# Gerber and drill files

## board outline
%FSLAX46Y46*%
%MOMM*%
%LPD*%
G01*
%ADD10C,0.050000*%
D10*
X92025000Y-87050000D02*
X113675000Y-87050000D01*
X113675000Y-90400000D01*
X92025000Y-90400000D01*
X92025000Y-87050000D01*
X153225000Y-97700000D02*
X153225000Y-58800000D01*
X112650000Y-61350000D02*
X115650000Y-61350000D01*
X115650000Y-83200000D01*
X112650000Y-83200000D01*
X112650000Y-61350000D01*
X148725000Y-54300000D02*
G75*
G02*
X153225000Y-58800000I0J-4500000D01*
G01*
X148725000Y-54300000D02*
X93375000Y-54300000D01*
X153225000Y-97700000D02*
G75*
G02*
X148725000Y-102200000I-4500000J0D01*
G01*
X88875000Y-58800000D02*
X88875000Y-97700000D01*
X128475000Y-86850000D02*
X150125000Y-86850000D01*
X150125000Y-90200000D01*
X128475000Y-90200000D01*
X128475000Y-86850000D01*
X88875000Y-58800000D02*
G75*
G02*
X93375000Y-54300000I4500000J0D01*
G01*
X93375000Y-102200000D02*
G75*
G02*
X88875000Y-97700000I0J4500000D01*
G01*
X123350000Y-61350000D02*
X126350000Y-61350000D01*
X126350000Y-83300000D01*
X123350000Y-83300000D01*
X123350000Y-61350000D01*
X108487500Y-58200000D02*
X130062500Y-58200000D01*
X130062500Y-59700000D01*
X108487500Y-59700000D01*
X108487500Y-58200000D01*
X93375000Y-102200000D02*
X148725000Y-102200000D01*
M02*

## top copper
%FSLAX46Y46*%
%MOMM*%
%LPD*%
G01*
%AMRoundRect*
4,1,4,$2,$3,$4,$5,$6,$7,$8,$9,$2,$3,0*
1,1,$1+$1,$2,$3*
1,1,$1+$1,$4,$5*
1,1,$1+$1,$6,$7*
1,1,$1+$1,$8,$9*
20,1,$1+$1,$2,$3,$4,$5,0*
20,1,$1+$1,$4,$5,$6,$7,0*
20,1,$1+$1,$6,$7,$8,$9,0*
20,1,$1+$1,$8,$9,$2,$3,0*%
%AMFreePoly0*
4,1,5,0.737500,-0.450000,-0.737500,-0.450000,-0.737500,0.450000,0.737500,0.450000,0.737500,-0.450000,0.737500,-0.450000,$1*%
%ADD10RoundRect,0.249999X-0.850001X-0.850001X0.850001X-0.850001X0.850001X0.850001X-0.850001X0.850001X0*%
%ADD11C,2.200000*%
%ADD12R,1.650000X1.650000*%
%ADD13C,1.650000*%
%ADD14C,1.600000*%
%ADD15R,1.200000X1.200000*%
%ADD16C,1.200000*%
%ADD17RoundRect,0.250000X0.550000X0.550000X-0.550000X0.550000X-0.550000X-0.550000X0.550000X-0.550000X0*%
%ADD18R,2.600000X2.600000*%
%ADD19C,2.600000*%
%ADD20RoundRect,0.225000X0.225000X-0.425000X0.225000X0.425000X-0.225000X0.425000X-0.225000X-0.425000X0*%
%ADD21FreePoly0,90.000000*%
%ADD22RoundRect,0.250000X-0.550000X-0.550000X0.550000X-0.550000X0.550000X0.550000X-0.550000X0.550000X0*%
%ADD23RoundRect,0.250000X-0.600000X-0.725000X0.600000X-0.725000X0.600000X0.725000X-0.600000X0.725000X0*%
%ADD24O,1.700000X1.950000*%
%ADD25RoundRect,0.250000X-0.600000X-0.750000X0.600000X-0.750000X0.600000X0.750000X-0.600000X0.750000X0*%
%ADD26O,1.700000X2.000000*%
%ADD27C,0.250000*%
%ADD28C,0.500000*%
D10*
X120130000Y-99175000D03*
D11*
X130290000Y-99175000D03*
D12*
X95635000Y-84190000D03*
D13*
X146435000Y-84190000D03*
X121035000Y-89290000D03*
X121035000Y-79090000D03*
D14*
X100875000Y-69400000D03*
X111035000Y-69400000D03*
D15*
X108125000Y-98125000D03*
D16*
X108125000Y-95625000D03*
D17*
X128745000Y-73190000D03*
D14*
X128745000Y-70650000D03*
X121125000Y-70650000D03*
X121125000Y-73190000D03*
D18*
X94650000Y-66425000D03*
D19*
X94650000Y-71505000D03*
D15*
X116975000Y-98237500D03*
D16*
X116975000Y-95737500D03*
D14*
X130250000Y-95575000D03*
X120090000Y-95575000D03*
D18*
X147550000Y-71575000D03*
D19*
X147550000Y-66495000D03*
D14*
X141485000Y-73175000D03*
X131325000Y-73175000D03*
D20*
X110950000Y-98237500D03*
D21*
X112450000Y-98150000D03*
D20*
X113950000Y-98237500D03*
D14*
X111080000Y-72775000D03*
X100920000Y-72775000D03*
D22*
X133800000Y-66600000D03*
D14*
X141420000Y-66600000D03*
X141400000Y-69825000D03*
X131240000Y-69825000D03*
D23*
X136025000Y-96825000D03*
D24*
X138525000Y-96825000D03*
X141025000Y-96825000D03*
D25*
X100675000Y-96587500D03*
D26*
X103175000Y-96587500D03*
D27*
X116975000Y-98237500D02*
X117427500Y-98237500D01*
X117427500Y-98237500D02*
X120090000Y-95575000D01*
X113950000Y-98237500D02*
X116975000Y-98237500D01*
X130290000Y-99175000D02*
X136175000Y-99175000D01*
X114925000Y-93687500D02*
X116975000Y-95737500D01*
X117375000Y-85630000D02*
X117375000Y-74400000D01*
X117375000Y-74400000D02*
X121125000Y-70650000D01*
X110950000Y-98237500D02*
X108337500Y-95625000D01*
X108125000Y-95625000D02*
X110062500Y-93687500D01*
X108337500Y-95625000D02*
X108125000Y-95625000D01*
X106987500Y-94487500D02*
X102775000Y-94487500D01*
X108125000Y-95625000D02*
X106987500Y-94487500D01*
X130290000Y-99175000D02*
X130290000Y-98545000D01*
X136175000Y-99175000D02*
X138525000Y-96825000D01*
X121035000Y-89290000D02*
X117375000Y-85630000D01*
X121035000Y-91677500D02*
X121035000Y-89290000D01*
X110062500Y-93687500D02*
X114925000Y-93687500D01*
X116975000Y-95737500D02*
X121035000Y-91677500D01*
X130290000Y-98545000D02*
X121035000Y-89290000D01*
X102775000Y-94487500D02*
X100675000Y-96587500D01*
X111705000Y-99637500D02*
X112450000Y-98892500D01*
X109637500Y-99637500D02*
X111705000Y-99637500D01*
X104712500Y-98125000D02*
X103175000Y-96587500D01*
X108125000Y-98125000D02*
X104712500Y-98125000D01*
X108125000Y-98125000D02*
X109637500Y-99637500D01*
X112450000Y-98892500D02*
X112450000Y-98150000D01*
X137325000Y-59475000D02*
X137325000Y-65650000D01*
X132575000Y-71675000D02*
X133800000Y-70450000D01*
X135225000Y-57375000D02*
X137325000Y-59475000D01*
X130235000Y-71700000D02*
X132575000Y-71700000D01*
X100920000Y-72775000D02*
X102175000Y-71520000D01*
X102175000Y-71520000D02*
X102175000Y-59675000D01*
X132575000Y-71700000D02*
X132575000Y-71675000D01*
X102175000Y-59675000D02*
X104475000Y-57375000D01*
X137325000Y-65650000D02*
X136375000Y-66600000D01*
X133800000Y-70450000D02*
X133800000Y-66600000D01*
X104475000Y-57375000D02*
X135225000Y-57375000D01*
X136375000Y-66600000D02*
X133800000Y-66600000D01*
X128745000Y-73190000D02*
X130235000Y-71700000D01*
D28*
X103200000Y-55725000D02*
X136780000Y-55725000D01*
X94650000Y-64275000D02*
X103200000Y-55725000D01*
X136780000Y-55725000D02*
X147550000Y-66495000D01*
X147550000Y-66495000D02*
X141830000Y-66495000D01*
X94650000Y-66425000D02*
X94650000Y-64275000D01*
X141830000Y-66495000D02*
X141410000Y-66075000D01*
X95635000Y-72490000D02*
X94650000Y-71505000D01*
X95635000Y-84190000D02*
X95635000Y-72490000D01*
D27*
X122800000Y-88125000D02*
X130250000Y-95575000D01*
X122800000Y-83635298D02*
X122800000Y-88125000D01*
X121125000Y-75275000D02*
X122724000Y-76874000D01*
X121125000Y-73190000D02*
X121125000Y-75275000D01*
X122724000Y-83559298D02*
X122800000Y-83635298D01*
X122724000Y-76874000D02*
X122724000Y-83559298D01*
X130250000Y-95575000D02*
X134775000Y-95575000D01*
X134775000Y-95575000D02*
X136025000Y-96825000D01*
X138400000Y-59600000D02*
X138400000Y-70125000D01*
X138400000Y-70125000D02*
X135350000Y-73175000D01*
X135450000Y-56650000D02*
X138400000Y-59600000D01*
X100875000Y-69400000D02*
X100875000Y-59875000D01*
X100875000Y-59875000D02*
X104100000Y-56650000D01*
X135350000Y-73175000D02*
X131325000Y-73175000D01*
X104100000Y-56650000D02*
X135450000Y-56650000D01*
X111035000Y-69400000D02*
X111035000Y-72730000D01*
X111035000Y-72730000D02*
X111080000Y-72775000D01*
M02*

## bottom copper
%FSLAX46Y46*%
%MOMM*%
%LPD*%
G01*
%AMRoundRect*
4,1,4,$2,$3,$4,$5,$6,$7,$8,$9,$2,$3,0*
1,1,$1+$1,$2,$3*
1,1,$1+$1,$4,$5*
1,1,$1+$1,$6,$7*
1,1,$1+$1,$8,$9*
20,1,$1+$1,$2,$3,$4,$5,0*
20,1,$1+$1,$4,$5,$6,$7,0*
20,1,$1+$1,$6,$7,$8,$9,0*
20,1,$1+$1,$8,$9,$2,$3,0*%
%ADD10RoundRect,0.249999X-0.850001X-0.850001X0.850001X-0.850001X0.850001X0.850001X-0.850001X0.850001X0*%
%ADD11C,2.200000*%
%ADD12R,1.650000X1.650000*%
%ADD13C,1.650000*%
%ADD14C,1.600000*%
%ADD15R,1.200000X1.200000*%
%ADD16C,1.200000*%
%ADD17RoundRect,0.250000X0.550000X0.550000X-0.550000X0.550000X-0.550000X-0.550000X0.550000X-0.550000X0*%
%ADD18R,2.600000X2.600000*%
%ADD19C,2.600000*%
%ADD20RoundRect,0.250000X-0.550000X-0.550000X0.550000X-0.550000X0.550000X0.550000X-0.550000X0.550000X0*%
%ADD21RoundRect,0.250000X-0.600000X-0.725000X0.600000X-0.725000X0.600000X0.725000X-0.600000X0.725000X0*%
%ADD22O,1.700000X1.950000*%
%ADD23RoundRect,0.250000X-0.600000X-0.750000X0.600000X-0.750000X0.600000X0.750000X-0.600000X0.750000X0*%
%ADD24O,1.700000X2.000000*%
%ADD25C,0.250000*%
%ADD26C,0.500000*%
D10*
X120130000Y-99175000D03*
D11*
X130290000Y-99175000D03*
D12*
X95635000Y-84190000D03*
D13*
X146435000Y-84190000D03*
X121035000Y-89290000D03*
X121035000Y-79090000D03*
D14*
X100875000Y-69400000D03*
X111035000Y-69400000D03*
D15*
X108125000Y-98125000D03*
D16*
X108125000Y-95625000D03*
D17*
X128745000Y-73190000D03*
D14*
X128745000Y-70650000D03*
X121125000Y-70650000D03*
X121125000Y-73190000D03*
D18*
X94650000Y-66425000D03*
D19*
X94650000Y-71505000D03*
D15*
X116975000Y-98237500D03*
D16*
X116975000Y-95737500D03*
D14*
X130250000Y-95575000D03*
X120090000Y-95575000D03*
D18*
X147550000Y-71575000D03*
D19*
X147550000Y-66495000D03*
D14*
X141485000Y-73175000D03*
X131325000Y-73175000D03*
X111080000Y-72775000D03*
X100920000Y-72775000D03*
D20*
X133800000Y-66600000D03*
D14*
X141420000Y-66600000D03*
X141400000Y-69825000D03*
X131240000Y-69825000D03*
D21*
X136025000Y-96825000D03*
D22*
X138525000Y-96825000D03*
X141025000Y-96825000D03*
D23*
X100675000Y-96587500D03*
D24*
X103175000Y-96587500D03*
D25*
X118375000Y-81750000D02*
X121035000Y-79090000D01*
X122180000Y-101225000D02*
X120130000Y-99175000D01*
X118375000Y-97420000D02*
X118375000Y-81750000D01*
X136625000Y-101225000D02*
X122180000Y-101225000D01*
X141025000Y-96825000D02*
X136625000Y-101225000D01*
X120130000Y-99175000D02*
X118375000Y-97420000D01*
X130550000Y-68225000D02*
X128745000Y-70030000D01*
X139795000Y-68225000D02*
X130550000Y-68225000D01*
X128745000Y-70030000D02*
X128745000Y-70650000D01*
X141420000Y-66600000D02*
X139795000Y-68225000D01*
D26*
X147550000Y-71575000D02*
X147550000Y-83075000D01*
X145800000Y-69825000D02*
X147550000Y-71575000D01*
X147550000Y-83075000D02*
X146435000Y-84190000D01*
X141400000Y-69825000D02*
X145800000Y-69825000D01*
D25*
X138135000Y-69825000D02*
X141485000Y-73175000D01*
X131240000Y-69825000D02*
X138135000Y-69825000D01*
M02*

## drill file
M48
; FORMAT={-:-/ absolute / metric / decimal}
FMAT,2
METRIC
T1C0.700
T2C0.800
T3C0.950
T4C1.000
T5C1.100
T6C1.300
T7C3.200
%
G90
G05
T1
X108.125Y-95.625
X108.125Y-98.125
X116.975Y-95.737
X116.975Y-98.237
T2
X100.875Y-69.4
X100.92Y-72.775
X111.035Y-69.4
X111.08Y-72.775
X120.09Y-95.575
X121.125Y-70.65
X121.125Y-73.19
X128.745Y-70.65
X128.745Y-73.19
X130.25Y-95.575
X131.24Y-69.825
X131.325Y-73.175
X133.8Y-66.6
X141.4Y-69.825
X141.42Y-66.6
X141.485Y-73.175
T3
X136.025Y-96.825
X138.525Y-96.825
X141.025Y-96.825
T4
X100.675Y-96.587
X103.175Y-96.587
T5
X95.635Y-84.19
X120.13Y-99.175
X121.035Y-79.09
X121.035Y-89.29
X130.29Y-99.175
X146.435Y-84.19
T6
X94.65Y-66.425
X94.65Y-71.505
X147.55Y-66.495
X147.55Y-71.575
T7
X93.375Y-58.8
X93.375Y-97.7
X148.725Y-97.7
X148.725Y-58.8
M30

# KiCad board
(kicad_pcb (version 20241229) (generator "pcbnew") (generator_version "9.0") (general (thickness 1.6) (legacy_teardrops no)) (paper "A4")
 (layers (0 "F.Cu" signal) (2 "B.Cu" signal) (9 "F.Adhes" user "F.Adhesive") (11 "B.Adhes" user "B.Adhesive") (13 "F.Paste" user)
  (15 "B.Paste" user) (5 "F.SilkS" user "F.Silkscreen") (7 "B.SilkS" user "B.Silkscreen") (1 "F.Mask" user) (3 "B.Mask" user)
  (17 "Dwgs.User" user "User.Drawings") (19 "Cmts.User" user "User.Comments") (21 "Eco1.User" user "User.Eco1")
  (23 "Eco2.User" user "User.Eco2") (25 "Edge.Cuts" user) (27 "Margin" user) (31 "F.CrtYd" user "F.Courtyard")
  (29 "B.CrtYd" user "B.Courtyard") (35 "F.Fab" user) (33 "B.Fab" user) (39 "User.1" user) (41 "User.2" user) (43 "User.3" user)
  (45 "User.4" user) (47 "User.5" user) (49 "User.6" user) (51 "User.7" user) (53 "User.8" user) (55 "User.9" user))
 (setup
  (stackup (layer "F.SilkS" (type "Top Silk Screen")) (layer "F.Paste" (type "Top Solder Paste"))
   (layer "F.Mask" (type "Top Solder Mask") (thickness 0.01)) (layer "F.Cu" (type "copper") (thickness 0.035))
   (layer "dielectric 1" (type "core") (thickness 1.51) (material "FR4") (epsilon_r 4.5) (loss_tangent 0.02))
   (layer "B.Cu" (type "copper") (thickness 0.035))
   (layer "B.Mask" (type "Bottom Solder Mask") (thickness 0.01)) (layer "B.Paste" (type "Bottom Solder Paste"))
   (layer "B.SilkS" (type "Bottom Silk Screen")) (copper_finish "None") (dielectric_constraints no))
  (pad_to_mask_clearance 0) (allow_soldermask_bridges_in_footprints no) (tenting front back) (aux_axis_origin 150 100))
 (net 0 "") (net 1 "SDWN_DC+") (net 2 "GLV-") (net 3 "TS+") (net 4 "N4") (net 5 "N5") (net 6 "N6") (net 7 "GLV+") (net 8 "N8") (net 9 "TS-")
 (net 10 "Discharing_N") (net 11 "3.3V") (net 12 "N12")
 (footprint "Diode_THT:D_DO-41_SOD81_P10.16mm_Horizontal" (layer "F.Cu") (at 120.13 99.175)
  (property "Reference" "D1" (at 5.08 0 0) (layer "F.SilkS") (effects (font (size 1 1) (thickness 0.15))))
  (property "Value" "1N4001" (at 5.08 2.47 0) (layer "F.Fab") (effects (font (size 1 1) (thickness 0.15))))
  (pad "1" thru_hole roundrect (at 0 0) (size 2.2 2.2) (drill 1.1) (layers "*.Cu" "*.Mask") (remove_unused_layers no)
   (roundrect_rratio 0.113636) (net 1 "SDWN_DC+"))
  (pad "2" thru_hole circle (at 10.16 0) (size 2.2 2.2) (drill 1.1) (layers "*.Cu" "*.Mask") (remove_unused_layers no) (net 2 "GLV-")))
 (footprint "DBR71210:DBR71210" (layer "F.Cu") (at 95.635 84.19)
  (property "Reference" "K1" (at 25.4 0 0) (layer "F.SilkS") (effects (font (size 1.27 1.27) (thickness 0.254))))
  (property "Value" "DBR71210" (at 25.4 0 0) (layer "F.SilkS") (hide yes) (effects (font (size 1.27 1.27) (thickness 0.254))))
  (pad "1" thru_hole rect (at 0 0) (size 1.65 1.65) (drill 1.1) (layers "*.Cu" "*.Mask") (remove_unused_layers no) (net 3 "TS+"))
  (pad "2" thru_hole circle (at 50.8 0) (size 1.65 1.65) (drill 1.1) (layers "*.Cu" "*.Mask") (remove_unused_layers no) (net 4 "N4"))
  (pad "3" thru_hole circle (at 25.4 5.1) (size 1.65 1.65) (drill 1.1) (layers "*.Cu" "*.Mask") (remove_unused_layers no) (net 2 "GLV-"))
  (pad "4" thru_hole circle (at 25.4 -5.1) (size 1.65 1.65) (drill 1.1) (layers "*.Cu" "*.Mask") (remove_unused_layers no)
   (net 1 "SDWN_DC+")))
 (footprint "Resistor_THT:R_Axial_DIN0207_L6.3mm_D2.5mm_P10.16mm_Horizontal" (layer "F.Cu") (at 100.875 69.4)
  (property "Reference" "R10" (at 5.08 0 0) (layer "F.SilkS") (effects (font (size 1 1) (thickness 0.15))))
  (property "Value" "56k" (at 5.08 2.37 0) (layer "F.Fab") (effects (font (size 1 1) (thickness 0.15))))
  (pad "1" thru_hole circle (at 0 0) (size 1.6 1.6) (drill 0.8) (layers "*.Cu" "*.Mask") (remove_unused_layers no) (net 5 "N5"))
  (pad "2" thru_hole circle (at 10.16 0) (size 1.6 1.6) (drill 0.8) (layers "*.Cu" "*.Mask") (remove_unused_layers no) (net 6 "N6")))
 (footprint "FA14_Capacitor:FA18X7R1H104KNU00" (layer "F.Cu") (at 108.125 98.125 90)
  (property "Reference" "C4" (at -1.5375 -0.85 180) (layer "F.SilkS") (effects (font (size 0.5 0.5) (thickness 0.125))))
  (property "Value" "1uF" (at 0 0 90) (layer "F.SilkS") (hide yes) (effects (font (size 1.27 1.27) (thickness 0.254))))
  (pad "1" thru_hole rect (at 0 0 90) (size 1.2 1.2) (drill 0.7) (layers "*.Cu" "*.Mask") (remove_unused_layers no) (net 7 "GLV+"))
  (pad "2" thru_hole circle (at 2.5 0 90) (size 1.2 1.2) (drill 0.7) (layers "*.Cu" "*.Mask") (remove_unused_layers no) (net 2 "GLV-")))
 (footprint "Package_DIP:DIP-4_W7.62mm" (layer "F.Cu") (at 128.745 73.19 180)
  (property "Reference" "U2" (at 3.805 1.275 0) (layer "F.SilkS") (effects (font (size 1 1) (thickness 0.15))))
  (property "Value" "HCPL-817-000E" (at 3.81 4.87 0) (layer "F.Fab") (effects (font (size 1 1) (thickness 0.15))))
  (pad "1" thru_hole roundrect (at 0 0 180) (size 1.6 1.6) (drill 0.8) (layers "*.Cu" "*.Mask") (remove_unused_layers no)
   (roundrect_rratio 0.15625) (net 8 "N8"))
  (pad "2" thru_hole circle (at 0 2.54 180) (size 1.6 1.6) (drill 0.8) (layers "*.Cu" "*.Mask") (remove_unused_layers no) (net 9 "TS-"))
  (pad "3" thru_hole circle (at 7.62 2.54 180) (size 1.6 1.6) (drill 0.8) (layers "*.Cu" "*.Mask") (remove_unused_layers no) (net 2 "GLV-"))
  (pad "4" thru_hole circle (at 7.62 0 180) (size 1.6 1.6) (drill 0.8) (layers "*.Cu" "*.Mask") (remove_unused_layers no)
   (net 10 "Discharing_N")))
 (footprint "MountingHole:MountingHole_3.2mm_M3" (layer "F.Cu") (at 93.374998 58.799998)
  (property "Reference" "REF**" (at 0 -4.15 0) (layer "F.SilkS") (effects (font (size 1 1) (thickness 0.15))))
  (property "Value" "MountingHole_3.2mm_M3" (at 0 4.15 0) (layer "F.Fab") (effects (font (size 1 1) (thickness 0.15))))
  (pad "" np_thru_hole circle (at 0 0) (size 3.2 3.2) (drill 3.2) (layers "*.Cu" "*.Mask")))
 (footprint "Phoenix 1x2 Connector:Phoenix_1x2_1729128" (layer "F.Cu") (at 94.65 66.425 -90)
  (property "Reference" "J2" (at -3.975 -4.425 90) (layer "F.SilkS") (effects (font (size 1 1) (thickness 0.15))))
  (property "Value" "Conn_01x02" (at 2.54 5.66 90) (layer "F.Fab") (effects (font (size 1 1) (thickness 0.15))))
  (pad "1" thru_hole rect (at 0 0 270) (size 2.6 2.6) (drill 1.3) (layers "*.Cu" "*.Mask") (remove_unused_layers no) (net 9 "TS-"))
  (pad "2" thru_hole circle (at 5.08 0 270) (size 2.6 2.6) (drill 1.3) (layers "*.Cu" "*.Mask") (remove_unused_layers no) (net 3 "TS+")))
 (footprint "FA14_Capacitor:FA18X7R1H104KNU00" (layer "F.Cu") (at 116.975 98.2375 90)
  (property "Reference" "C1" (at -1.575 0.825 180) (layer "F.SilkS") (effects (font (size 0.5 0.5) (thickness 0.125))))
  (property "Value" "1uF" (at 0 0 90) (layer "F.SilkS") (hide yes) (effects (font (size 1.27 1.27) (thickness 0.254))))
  (pad "1" thru_hole rect (at 0 0 90) (size 1.2 1.2) (drill 0.7) (layers "*.Cu" "*.Mask") (remove_unused_layers no) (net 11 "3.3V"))
  (pad "2" thru_hole circle (at 2.5 0 90) (size 1.2 1.2) (drill 0.7) (layers "*.Cu" "*.Mask") (remove_unused_layers no) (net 2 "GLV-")))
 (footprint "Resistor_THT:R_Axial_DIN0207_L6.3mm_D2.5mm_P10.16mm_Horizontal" (layer "F.Cu") (at 130.25 95.575 180)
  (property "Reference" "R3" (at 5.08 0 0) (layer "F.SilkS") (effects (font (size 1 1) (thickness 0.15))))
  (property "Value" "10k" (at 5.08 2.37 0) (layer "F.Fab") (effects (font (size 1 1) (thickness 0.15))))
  (pad "1" thru_hole circle (at 0 0 180) (size 1.6 1.6) (drill 0.8) (layers "*.Cu" "*.Mask") (remove_unused_layers no)
   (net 10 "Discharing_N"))
  (pad "2" thru_hole circle (at 10.16 0 180) (size 1.6 1.6) (drill 0.8) (layers "*.Cu" "*.Mask") (remove_unused_layers no) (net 11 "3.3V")))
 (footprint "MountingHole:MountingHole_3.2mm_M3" (layer "F.Cu") (at 148.725002 58.799998)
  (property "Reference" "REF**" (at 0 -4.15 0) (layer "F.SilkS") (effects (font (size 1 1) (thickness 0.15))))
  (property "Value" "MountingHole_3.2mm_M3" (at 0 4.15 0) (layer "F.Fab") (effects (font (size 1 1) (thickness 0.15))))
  (pad "" np_thru_hole circle (at 0 0) (size 3.2 3.2) (drill 3.2) (layers "*.Cu" "*.Mask")))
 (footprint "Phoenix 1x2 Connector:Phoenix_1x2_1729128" (layer "F.Cu") (at 147.55 71.575 90)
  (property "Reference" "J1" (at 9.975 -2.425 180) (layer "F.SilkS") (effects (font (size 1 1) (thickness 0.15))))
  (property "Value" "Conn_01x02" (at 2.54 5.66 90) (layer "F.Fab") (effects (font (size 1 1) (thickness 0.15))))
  (pad "1" thru_hole rect (at 0 0 90) (size 2.6 2.6) (drill 1.3) (layers "*.Cu" "*.Mask") (remove_unused_layers no) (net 4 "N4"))
  (pad "2" thru_hole circle (at 5.08 0 90) (size 2.6 2.6) (drill 1.3) (layers "*.Cu" "*.Mask") (remove_unused_layers no) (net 9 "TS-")))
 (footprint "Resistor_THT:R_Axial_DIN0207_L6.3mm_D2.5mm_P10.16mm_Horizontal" (layer "F.Cu") (at 141.485 73.175 180)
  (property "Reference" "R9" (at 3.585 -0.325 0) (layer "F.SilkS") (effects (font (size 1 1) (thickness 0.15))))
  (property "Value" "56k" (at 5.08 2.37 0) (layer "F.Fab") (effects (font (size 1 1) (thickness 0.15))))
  (pad "1" thru_hole circle (at 0 0 180) (size 1.6 1.6) (drill 0.8) (layers "*.Cu" "*.Mask") (remove_unused_layers no) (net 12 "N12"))
  (pad "2" thru_hole circle (at 10.16 0 180) (size 1.6 1.6) (drill 0.8) (layers "*.Cu" "*.Mask") (remove_unused_layers no) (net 5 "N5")))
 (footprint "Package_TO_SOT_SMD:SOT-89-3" (layer "F.Cu") (at 112.45 96.2875 90)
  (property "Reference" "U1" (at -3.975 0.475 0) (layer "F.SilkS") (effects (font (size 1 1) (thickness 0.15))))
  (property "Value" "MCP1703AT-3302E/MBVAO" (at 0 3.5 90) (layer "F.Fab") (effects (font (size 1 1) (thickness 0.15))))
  (pad "1" smd roundrect (at -1.95 -1.5 90) (size 1.3 0.9) (layers "F.Cu" "F.Mask" "F.Paste") (roundrect_rratio 0.25) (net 2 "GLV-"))
  (pad "2" smd custom (at -1.8625 0 90) (size 1.475 0.9) (layers "F.Cu" "F.Mask" "F.Paste") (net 7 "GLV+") (zone_connect 2)
   (thermal_bridge_angle 45) (options (clearance outline) (anchor rect)) (primitives))
  (pad "3" smd roundrect (at -1.95 1.5 90) (size 1.3 0.9) (layers "F.Cu" "F.Mask" "F.Paste") (roundrect_rratio 0.25) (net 11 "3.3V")))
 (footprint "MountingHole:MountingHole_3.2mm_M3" (layer "F.Cu") (at 93.375 97.7)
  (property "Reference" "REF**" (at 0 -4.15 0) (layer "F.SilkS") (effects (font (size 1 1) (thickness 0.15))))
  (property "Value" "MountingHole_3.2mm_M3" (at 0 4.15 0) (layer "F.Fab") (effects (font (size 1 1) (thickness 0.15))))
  (pad "" np_thru_hole circle (at 0 0) (size 3.2 3.2) (drill 3.2) (layers "*.Cu" "*.Mask")))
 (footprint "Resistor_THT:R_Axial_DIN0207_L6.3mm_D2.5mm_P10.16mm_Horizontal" (layer "F.Cu") (at 111.08 72.775 180)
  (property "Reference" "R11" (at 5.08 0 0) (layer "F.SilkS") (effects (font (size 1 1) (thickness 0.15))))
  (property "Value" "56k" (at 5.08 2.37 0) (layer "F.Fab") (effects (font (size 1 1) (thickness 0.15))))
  (pad "1" thru_hole circle (at 0 0 180) (size 1.6 1.6) (drill 0.8) (layers "*.Cu" "*.Mask") (remove_unused_layers no) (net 6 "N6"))
  (pad "2" thru_hole circle (at 10.16 0 180) (size 1.6 1.6) (drill 0.8) (layers "*.Cu" "*.Mask") (remove_unused_layers no) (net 8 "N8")))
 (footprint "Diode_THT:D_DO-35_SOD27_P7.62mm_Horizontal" (layer "F.Cu") (at 133.8 66.6)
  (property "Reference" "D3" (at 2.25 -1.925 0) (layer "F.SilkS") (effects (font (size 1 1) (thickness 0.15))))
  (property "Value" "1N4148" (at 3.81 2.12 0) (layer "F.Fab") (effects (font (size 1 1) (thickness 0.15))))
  (pad "1" thru_hole roundrect (at 0 0) (size 1.6 1.6) (drill 0.8) (layers "*.Cu" "*.Mask") (remove_unused_layers no)
   (roundrect_rratio 0.15625) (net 8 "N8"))
  (pad "2" thru_hole circle (at 7.62 0) (size 1.6 1.6) (drill 0.8) (layers "*.Cu" "*.Mask") (remove_unused_layers no) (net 9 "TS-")))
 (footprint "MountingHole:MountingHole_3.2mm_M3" (layer "F.Cu") (at 148.725 97.700002)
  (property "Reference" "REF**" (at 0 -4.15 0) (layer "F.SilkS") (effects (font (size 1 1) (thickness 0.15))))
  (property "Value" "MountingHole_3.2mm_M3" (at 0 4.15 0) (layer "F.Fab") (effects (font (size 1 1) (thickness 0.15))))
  (pad "" np_thru_hole circle (at 0 0) (size 3.2 3.2) (drill 3.2) (layers "*.Cu" "*.Mask")))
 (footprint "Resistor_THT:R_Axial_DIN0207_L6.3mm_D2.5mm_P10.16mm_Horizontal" (layer "F.Cu") (at 141.4 69.825 180)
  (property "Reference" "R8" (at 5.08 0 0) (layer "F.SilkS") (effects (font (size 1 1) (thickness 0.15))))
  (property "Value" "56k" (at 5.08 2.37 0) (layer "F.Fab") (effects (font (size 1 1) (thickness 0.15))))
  (pad "1" thru_hole circle (at 0 0 180) (size 1.6 1.6) (drill 0.8) (layers "*.Cu" "*.Mask") (remove_unused_layers no) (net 4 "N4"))
  (pad "2" thru_hole circle (at 10.16 0 180) (size 1.6 1.6) (drill 0.8) (layers "*.Cu" "*.Mask") (remove_unused_layers no) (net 12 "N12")))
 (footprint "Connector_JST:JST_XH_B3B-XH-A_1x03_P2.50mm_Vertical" (layer "F.Cu") (at 136.025 96.825)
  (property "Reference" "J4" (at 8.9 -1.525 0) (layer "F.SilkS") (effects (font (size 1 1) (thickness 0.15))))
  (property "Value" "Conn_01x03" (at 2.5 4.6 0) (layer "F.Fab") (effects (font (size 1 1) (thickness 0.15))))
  (pad "1" thru_hole roundrect (at 0 0) (size 1.7 1.95) (drill 0.95) (layers "*.Cu" "*.Mask") (remove_unused_layers no)
   (roundrect_rratio 0.147059) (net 10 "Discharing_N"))
  (pad "2" thru_hole oval (at 2.5 0) (size 1.7 1.95) (drill 0.95) (layers "*.Cu" "*.Mask") (remove_unused_layers no) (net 2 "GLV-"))
  (pad "3" thru_hole oval (at 5 0) (size 1.7 1.95) (drill 0.95) (layers "*.Cu" "*.Mask") (remove_unused_layers no) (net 1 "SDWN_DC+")))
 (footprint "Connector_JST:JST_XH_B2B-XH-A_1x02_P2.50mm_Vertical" (layer "F.Cu") (at 100.675 96.5875)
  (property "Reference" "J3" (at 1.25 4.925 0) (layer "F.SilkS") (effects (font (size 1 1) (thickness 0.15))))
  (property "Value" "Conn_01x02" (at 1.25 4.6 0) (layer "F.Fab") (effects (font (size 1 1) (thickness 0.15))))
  (pad "1" thru_hole roundrect (at 0 0) (size 1.7 2) (drill 1) (layers "*.Cu" "*.Mask") (remove_unused_layers no)
   (roundrect_rratio 0.147059) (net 2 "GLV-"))
  (pad "2" thru_hole oval (at 2.5 0) (size 1.7 2) (drill 1) (layers "*.Cu" "*.Mask") (remove_unused_layers no) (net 7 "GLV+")))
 (gr_rect (start 92.025 87.05) (end 113.675 90.4) (stroke (width 0.05) (type default)) (fill no) (layer "Edge.Cuts"))
 (gr_line (start 153.225 97.7) (end 153.225 58.8) (stroke (width 0.05) (type default)) (layer "Edge.Cuts"))
 (gr_rect (start 112.65 61.35) (end 115.65 83.2) (stroke (width 0.05) (type default)) (fill no) (layer "Edge.Cuts"))
 (gr_arc (start 148.725 54.3) (mid 151.906981 55.618019) (end 153.225 58.8) (stroke (width 0.05) (type default)) (layer "Edge.Cuts"))
 (gr_line (start 148.725 54.3) (end 93.375 54.3) (stroke (width 0.05) (type default)) (layer "Edge.Cuts"))
 (gr_arc (start 153.225 97.7) (mid 151.906981 100.881981) (end 148.725 102.2) (stroke (width 0.05) (type default)) (layer "Edge.Cuts"))
 (gr_line (start 88.875 58.8) (end 88.875 97.7) (stroke (width 0.05) (type default)) (layer "Edge.Cuts"))
 (gr_rect (start 128.475 86.85) (end 150.125 90.2) (stroke (width 0.05) (type default)) (fill no) (layer "Edge.Cuts"))
 (gr_arc (start 88.875 58.8) (mid 90.193019 55.618019) (end 93.375 54.3) (stroke (width 0.05) (type default)) (layer "Edge.Cuts"))
 (gr_arc (start 93.375 102.2) (mid 90.193019 100.881981) (end 88.875 97.7) (stroke (width 0.05) (type default)) (layer "Edge.Cuts"))
 (gr_rect (start 123.35 61.35) (end 126.35 83.3) (stroke (width 0.05) (type default)) (fill no) (layer "Edge.Cuts"))
 (gr_rect (start 108.4875 58.2) (end 130.0625 59.7) (stroke (width 0.05) (type default)) (fill no) (layer "Edge.Cuts"))
 (gr_line (start 93.375 102.2) (end 148.725 102.2) (stroke (width 0.05) (type default)) (layer "Edge.Cuts"))
 (segment (start 116.975 98.2375) (end 117.4275 98.2375) (width 0.25) (layer "F.Cu") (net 11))
 (segment (start 117.4275 98.2375) (end 120.09 95.575) (width 0.25) (layer "F.Cu") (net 11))
 (segment (start 113.95 98.2375) (end 116.975 98.2375) (width 0.25) (layer "F.Cu") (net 11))
 (segment (start 130.29 99.175) (end 136.175 99.175) (width 0.25) (layer "F.Cu") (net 2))
 (segment (start 114.925 93.6875) (end 116.975 95.7375) (width 0.25) (layer "F.Cu") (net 2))
 (segment (start 117.375 85.63) (end 117.375 74.4) (width 0.25) (layer "F.Cu") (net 2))
 (segment (start 117.375 74.4) (end 121.125 70.65) (width 0.25) (layer "F.Cu") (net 2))
 (segment (start 110.95 98.2375) (end 108.3375 95.625) (width 0.25) (layer "F.Cu") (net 2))
 (segment (start 108.125 95.625) (end 110.0625 93.6875) (width 0.25) (layer "F.Cu") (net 2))
 (segment (start 108.3375 95.625) (end 108.125 95.625) (width 0.25) (layer "F.Cu") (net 2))
 (segment (start 106.9875 94.4875) (end 102.775 94.4875) (width 0.25) (layer "F.Cu") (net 2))
 (segment (start 108.125 95.625) (end 106.9875 94.4875) (width 0.25) (layer "F.Cu") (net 2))
 (segment (start 130.29 99.175) (end 130.29 98.545) (width 0.25) (layer "F.Cu") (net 2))
 (segment (start 136.175 99.175) (end 138.525 96.825) (width 0.25) (layer "F.Cu") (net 2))
 (segment (start 121.035 89.29) (end 117.375 85.63) (width 0.25) (layer "F.Cu") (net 2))
 (segment (start 121.035 91.6775) (end 121.035 89.29) (width 0.25) (layer "F.Cu") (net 2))
 (segment (start 110.0625 93.6875) (end 114.925 93.6875) (width 0.25) (layer "F.Cu") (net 2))
 (segment (start 116.975 95.7375) (end 121.035 91.6775) (width 0.25) (layer "F.Cu") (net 2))
 (segment (start 130.29 98.545) (end 121.035 89.29) (width 0.25) (layer "F.Cu") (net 2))
 (segment (start 102.775 94.4875) (end 100.675 96.5875) (width 0.25) (layer "F.Cu") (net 2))
 (segment (start 111.705 99.6375) (end 112.45 98.8925) (width 0.25) (layer "F.Cu") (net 7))
 (segment (start 109.6375 99.6375) (end 111.705 99.6375) (width 0.25) (layer "F.Cu") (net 7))
 (segment (start 104.7125 98.125) (end 103.175 96.5875) (width 0.25) (layer "F.Cu") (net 7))
 (segment (start 108.125 98.125) (end 104.7125 98.125) (width 0.25) (layer "F.Cu") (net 7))
 (segment (start 108.125 98.125) (end 109.6375 99.6375) (width 0.25) (layer "F.Cu") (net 7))
 (segment (start 112.45 98.8925) (end 112.45 98.15) (width 0.25) (layer "F.Cu") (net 7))
 (segment (start 118.375 81.75) (end 121.035 79.09) (width 0.25) (layer "B.Cu") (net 1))
 (segment (start 122.18 101.225) (end 120.13 99.175) (width 0.25) (layer "B.Cu") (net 1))
 (segment (start 118.375 97.42) (end 118.375 81.75) (width 0.25) (layer "B.Cu") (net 1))
 (segment (start 136.625 101.225) (end 122.18 101.225) (width 0.25) (layer "B.Cu") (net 1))
 (segment (start 141.025 96.825) (end 136.625 101.225) (width 0.25) (layer "B.Cu") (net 1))
 (segment (start 120.13 99.175) (end 118.375 97.42) (width 0.25) (layer "B.Cu") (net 1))
 (segment (start 137.325 59.475) (end 137.325 65.65) (width 0.25) (layer "F.Cu") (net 8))
 (segment (start 132.575 71.675) (end 133.8 70.45) (width 0.25) (layer "F.Cu") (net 8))
 (segment (start 135.225 57.375) (end 137.325 59.475) (width 0.25) (layer "F.Cu") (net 8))
 (segment (start 130.235 71.7) (end 132.575 71.7) (width 0.25) (layer "F.Cu") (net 8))
 (segment (start 100.92 72.775) (end 102.175 71.52) (width 0.25) (layer "F.Cu") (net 8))
 (segment (start 102.175 71.52) (end 102.175 59.675) (width 0.25) (layer "F.Cu") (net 8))
 (segment (start 132.575 71.7) (end 132.575 71.675) (width 0.25) (layer "F.Cu") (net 8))
 (segment (start 102.175 59.675) (end 104.475 57.375) (width 0.25) (layer "F.Cu") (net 8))
 (segment (start 137.325 65.65) (end 136.375 66.6) (width 0.25) (layer "F.Cu") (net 8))
 (segment (start 133.8 70.45) (end 133.8 66.6) (width 0.25) (layer "F.Cu") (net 8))
 (segment (start 104.475 57.375) (end 135.225 57.375) (width 0.25) (layer "F.Cu") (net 8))
 (segment (start 136.375 66.6) (end 133.8 66.6) (width 0.25) (layer "F.Cu") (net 8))
 (segment (start 128.745 73.19) (end 130.235 71.7) (width 0.25) (layer "F.Cu") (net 8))
 (segment (start 103.2 55.725) (end 136.78 55.725) (width 0.5) (layer "F.Cu") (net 9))
 (segment (start 94.65 64.275) (end 103.2 55.725) (width 0.5) (layer "F.Cu") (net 9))
 (segment (start 136.78 55.725) (end 147.55 66.495) (width 0.5) (layer "F.Cu") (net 9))
 (segment (start 147.55 66.495) (end 141.83 66.495) (width 0.5) (layer "F.Cu") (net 9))
 (segment (start 94.65 66.425) (end 94.65 64.275) (width 0.5) (layer "F.Cu") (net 9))
 (segment (start 141.83 66.495) (end 141.41 66.075) (width 0.5) (layer "F.Cu") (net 9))
 (segment (start 130.55 68.225) (end 128.745 70.03) (width 0.25) (layer "B.Cu") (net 9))
 (segment (start 139.795 68.225) (end 130.55 68.225) (width 0.25) (layer "B.Cu") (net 9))
 (segment (start 128.745 70.03) (end 128.745 70.65) (width 0.25) (layer "B.Cu") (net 9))
 (segment (start 141.42 66.6) (end 139.795 68.225) (width 0.25) (layer "B.Cu") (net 9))
 (segment (start 147.55 71.575) (end 147.55 83.075) (width 0.5) (layer "B.Cu") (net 4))
 (segment (start 145.8 69.825) (end 147.55 71.575) (width 0.5) (layer "B.Cu") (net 4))
 (segment (start 147.55 83.075) (end 146.435 84.19) (width 0.5) (layer "B.Cu") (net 4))
 (segment (start 141.4 69.825) (end 145.8 69.825) (width 0.5) (layer "B.Cu") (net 4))
 (segment (start 95.635 72.49) (end 94.65 71.505) (width 0.5) (layer "F.Cu") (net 3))
 (segment (start 95.635 84.19) (end 95.635 72.49) (width 0.5) (layer "F.Cu") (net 3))
 (segment (start 122.8 88.125) (end 130.25 95.575) (width 0.25) (layer "F.Cu") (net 10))
 (segment (start 122.8 83.635298) (end 122.8 88.125) (width 0.25) (layer "F.Cu") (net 10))
 (segment (start 121.125 75.275) (end 122.724 76.874) (width 0.25) (layer "F.Cu") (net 10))
 (segment (start 121.125 73.19) (end 121.125 75.275) (width 0.25) (layer "F.Cu") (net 10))
 (segment (start 122.724 83.559298) (end 122.8 83.635298) (width 0.25) (layer "F.Cu") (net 10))
 (segment (start 122.724 76.874) (end 122.724 83.559298) (width 0.25) (layer "F.Cu") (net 10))
 (segment (start 130.25 95.575) (end 134.775 95.575) (width 0.25) (layer "F.Cu") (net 10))
 (segment (start 134.775 95.575) (end 136.025 96.825) (width 0.25) (layer "F.Cu") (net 10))
 (segment (start 138.135 69.825) (end 141.485 73.175) (width 0.25) (layer "B.Cu") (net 12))
 (segment (start 131.24 69.825) (end 138.135 69.825) (width 0.25) (layer "B.Cu") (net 12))
 (segment (start 138.4 59.6) (end 138.4 70.125) (width 0.25) (layer "F.Cu") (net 5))
 (segment (start 138.4 70.125) (end 135.35 73.175) (width 0.25) (layer "F.Cu") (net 5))
 (segment (start 135.45 56.65) (end 138.4 59.6) (width 0.25) (layer "F.Cu") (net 5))
 (segment (start 100.875 69.4) (end 100.875 59.875) (width 0.25) (layer "F.Cu") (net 5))
 (segment (start 100.875 59.875) (end 104.1 56.65) (width 0.25) (layer "F.Cu") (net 5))
 (segment (start 135.35 73.175) (end 131.325 73.175) (width 0.25) (layer "F.Cu") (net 5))
 (segment (start 104.1 56.65) (end 135.45 56.65) (width 0.25) (layer "F.Cu") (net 5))
 (segment (start 111.035 69.4) (end 111.035 72.73) (width 0.25) (layer "F.Cu") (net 6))
 (segment (start 111.035 72.73) (end 111.08 72.775) (width 0.25) (layer "F.Cu") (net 6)))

